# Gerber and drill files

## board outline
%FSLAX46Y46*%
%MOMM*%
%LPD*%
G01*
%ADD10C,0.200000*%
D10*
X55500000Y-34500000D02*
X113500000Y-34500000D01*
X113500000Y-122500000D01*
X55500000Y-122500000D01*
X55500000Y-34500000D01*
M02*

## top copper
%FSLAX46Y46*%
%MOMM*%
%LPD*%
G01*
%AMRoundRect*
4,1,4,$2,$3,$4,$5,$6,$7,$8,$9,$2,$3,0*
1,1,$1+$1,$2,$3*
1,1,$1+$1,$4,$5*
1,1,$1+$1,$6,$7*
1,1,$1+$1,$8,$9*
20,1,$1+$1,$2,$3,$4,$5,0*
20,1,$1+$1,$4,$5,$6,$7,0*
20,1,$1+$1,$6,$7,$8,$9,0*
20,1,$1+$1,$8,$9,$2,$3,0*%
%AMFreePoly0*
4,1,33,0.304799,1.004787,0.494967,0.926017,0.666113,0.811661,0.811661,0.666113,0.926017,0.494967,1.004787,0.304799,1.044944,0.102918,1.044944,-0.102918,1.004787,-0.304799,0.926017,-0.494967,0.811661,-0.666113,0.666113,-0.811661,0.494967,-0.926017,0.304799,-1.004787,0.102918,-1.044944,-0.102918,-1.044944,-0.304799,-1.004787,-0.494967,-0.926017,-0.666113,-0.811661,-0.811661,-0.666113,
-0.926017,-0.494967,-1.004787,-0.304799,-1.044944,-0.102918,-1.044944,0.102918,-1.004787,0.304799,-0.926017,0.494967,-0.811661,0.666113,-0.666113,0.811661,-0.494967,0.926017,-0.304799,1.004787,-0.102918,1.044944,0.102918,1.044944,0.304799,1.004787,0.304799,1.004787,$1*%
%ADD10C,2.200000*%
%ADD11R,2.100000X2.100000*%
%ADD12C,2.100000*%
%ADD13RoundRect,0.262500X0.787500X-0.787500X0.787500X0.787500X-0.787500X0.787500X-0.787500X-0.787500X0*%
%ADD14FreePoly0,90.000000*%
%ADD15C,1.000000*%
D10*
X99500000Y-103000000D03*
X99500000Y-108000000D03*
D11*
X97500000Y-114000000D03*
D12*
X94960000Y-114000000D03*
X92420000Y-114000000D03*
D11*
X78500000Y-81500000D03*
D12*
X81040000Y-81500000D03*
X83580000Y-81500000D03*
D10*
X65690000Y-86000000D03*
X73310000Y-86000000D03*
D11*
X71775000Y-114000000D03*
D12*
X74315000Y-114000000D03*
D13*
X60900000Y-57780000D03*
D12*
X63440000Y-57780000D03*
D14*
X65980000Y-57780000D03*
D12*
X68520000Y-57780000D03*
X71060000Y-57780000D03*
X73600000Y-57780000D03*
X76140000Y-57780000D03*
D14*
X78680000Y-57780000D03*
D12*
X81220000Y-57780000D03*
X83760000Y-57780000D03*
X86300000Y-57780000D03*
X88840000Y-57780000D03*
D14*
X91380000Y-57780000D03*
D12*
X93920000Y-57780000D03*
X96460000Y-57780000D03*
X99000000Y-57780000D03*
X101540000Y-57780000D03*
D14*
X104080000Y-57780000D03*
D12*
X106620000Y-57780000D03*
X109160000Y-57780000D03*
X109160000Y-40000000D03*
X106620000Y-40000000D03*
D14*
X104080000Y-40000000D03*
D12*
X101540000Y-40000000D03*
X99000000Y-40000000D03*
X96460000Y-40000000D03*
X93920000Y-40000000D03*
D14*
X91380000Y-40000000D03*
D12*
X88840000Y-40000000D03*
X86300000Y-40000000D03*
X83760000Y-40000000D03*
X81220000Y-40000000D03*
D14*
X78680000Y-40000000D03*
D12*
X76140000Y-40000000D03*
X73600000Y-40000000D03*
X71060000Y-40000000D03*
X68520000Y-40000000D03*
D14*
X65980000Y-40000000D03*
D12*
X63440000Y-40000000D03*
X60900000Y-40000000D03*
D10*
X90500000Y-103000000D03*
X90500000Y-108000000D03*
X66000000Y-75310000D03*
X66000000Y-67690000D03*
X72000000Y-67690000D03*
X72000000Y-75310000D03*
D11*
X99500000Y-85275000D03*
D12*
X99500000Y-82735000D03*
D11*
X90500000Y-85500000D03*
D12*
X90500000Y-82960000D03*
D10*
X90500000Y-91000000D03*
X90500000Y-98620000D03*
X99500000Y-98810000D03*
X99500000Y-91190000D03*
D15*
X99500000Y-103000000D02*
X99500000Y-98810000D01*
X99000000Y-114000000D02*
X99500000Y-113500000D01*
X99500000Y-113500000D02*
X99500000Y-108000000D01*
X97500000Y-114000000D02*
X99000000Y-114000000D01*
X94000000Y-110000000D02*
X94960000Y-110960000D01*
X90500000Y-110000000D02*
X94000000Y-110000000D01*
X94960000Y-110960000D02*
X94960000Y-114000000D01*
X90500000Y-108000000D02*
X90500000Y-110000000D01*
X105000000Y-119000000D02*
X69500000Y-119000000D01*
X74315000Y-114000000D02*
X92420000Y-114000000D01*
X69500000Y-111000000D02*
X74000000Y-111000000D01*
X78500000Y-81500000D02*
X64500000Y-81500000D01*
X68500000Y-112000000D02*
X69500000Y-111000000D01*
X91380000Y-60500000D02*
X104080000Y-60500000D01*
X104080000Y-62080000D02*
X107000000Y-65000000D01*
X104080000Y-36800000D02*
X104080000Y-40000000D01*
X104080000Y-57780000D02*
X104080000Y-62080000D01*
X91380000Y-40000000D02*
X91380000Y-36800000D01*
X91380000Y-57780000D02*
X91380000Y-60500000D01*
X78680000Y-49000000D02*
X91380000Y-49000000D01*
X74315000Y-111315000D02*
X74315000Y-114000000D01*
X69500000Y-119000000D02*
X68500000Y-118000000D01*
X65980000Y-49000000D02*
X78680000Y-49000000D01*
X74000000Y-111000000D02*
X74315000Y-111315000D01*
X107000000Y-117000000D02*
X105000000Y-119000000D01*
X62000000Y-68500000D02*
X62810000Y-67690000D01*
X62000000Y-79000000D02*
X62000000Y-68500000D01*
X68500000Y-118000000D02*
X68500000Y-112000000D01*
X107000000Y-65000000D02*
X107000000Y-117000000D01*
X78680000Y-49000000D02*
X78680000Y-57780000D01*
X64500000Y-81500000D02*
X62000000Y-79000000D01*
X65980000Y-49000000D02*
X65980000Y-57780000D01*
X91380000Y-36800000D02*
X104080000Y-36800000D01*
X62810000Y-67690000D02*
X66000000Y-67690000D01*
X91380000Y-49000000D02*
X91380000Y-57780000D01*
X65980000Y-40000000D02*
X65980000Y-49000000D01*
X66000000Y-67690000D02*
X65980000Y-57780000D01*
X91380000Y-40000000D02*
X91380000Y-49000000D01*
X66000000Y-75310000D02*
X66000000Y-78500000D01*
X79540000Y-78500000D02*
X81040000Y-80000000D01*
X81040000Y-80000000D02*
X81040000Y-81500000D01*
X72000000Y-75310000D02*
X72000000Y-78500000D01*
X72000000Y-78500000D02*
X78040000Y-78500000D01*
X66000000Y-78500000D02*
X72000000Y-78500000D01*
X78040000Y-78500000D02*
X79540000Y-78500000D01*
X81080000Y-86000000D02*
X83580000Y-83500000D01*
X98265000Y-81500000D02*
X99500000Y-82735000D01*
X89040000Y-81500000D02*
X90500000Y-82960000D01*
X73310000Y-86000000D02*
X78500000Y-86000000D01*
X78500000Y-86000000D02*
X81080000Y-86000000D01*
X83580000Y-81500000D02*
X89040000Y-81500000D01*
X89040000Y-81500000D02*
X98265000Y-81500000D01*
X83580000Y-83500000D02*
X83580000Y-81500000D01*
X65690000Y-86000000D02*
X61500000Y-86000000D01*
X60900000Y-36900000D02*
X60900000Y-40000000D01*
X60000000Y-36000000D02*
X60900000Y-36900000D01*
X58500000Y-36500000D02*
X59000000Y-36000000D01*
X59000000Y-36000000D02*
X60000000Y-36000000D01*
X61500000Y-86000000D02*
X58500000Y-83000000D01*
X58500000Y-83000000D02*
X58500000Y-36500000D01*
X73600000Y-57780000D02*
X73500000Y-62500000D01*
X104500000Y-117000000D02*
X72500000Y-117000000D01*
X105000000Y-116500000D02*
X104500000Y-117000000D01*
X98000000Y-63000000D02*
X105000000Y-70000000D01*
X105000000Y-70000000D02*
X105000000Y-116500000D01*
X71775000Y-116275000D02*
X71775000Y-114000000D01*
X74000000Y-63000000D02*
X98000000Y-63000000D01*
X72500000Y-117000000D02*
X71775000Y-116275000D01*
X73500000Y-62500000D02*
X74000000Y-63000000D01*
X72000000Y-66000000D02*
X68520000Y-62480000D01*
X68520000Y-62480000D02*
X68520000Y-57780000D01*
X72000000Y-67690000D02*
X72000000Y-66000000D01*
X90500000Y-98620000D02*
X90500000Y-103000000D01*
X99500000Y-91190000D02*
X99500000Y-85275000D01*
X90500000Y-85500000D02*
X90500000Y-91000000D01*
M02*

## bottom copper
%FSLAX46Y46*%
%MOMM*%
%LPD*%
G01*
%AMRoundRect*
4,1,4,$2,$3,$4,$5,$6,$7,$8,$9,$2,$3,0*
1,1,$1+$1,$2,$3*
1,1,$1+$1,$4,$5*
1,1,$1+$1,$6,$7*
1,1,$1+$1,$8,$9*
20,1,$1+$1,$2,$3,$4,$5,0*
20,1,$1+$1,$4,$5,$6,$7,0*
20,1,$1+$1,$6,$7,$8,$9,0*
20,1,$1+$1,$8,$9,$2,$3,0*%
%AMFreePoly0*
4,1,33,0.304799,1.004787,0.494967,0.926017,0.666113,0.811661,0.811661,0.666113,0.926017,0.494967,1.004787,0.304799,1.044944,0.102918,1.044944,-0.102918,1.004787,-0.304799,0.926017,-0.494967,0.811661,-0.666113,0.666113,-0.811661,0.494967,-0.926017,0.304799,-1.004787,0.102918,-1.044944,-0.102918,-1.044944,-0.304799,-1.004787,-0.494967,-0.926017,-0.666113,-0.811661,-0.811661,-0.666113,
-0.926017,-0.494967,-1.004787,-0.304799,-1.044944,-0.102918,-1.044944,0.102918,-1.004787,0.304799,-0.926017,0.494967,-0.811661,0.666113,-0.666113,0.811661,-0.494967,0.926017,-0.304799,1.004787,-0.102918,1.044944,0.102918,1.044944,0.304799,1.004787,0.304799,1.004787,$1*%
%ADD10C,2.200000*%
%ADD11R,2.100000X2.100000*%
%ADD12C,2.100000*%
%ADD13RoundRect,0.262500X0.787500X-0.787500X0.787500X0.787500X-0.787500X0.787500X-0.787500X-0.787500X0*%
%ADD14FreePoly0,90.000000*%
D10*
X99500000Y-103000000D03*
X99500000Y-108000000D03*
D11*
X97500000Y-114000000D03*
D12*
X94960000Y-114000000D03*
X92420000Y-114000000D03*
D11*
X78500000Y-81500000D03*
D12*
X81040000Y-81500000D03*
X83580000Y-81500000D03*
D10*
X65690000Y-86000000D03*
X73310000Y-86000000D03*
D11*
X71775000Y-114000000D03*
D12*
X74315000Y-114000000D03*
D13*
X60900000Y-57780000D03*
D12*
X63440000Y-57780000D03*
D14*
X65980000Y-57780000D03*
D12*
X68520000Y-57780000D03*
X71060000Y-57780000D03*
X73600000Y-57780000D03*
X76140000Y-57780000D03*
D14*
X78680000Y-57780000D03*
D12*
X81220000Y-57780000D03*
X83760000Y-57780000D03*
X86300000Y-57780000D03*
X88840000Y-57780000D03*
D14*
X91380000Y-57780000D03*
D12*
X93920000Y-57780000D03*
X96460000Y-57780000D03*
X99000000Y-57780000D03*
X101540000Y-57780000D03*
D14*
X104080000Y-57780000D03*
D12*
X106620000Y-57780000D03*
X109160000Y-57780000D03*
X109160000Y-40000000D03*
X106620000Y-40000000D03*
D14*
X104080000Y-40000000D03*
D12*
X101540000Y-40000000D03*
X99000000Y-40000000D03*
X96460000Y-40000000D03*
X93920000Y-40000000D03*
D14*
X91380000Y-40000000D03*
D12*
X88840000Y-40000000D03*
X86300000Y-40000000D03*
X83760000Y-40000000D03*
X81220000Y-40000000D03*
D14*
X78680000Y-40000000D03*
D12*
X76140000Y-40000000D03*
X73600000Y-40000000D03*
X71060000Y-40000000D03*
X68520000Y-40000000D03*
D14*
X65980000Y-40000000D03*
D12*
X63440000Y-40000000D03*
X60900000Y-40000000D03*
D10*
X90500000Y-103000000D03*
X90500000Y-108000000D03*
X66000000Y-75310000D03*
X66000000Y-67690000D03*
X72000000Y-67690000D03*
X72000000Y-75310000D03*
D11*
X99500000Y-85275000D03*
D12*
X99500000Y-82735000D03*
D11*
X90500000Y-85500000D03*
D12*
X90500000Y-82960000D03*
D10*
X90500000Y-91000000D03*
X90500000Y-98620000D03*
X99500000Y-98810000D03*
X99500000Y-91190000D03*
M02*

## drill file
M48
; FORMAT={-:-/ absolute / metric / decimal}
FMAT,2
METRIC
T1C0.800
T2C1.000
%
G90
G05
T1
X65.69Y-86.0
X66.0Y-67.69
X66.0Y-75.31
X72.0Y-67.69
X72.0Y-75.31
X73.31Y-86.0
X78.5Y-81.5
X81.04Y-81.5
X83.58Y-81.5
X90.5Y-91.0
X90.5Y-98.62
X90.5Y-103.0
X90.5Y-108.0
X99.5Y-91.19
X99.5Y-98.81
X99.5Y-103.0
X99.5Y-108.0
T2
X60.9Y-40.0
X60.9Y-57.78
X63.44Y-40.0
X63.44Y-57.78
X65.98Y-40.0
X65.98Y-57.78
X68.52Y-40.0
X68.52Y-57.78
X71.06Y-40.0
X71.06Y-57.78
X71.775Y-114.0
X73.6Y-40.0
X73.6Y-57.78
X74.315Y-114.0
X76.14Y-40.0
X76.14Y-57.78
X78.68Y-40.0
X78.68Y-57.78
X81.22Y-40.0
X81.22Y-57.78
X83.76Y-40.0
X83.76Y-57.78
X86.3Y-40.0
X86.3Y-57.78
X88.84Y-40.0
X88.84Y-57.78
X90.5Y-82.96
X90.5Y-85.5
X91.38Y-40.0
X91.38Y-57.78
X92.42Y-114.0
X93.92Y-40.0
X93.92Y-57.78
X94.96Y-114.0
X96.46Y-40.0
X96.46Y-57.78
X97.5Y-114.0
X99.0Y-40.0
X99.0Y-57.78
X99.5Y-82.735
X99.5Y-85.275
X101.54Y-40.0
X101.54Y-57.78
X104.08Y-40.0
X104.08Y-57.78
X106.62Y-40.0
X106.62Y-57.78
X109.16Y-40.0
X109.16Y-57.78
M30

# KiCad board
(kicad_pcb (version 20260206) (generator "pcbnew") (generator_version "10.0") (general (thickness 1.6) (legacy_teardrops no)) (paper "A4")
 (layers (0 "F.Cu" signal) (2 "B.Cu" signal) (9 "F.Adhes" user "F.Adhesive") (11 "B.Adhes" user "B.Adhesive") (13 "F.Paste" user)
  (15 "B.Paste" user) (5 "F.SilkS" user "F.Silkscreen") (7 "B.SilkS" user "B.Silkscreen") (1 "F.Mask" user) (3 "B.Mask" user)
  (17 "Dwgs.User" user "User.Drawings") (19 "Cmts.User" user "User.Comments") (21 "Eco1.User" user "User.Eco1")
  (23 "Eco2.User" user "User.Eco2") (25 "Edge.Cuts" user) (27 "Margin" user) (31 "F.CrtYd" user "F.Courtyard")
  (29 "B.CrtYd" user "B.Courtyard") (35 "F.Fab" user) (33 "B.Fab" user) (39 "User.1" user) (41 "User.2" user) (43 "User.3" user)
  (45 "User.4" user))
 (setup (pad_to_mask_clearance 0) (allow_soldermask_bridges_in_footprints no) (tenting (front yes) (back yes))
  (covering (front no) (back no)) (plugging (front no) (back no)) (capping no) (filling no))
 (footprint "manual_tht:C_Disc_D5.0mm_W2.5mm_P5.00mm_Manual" (layer "F.Cu") (at 99.5 103 -90)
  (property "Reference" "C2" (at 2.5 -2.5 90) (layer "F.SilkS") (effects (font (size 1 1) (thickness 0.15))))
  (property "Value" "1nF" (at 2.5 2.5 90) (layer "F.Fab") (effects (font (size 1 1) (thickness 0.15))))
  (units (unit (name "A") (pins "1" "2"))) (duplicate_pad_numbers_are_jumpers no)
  (pad "1" thru_hole circle (at 0 0 270) (size 2.2 2.2) (drill 0.8) (layers "*.Cu" "*.Mask") (remove_unused_layers no) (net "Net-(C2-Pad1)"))
  (pad "2" thru_hole circle (at 5 0 270) (size 2.2 2.2) (drill 0.8) (layers "*.Cu" "*.Mask") (remove_unused_layers no) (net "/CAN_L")))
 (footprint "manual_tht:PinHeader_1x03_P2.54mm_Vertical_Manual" (layer "F.Cu") (at 97.5 114 -90)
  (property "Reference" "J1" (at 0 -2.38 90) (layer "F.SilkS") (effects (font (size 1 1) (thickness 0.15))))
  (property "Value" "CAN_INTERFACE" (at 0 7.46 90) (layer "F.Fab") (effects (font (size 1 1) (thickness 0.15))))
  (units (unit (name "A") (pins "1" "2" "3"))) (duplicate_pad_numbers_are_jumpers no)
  (pad "1" thru_hole rect (at 0 0 270) (size 2.1 2.1) (drill 1) (layers "*.Cu" "*.Mask") (remove_unused_layers no) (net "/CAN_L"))
  (pad "2" thru_hole circle (at 0 2.54 270) (size 2.1 2.1) (drill 1) (layers "*.Cu" "*.Mask") (remove_unused_layers no) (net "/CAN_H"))
  (pad "3" thru_hole circle (at 0 5.08 270) (size 2.1 2.1) (drill 1) (layers "*.Cu" "*.Mask") (remove_unused_layers no) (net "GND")))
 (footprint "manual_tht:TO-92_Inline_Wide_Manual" (layer "F.Cu") (at 78.5 81.5)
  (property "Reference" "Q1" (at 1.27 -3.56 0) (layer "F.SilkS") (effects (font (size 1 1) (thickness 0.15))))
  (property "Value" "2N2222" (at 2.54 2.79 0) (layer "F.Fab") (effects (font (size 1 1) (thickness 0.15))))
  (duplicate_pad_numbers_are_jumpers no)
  (pad "1" thru_hole rect (at 0 0) (size 2.1 2.1) (drill 0.8) (layers "*.Cu" "*.Mask") (remove_unused_layers no) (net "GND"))
  (pad "2" thru_hole circle (at 2.54 0) (size 2.1 2.1) (drill 0.8) (layers "*.Cu" "*.Mask") (remove_unused_layers no) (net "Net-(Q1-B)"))
  (pad "3" thru_hole circle (at 5.08 0) (size 2.1 2.1) (drill 0.8) (layers "*.Cu" "*.Mask") (remove_unused_layers no) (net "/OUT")))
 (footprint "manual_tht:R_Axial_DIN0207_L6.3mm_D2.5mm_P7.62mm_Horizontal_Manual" (layer "F.Cu") (at 65.69 86)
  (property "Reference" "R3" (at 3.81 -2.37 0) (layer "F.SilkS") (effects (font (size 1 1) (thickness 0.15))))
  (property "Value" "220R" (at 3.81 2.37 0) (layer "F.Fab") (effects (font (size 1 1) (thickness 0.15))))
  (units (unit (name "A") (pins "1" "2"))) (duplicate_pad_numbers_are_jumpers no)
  (pad "1" thru_hole circle (at 0 0) (size 2.2 2.2) (drill 0.8) (layers "*.Cu" "*.Mask") (remove_unused_layers no) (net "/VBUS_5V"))
  (pad "2" thru_hole circle (at 7.62 0) (size 2.2 2.2) (drill 0.8) (layers "*.Cu" "*.Mask") (remove_unused_layers no) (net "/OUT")))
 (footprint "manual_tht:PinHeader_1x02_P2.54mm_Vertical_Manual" (layer "F.Cu") (at 71.775 114 90)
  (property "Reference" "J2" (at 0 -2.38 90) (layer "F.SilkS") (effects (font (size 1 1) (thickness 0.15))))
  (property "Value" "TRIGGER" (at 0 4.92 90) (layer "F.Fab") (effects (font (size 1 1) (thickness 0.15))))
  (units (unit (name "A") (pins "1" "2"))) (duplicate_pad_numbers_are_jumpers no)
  (pad "1" thru_hole rect (at 0 0 90) (size 2.1 2.1) (drill 1) (layers "*.Cu" "*.Mask") (remove_unused_layers no) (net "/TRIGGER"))
  (pad "2" thru_hole circle (at 0 2.54 90) (size 2.1 2.1) (drill 1) (layers "*.Cu" "*.Mask") (remove_unused_layers no) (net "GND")))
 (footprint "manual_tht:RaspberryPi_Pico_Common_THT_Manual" (layer "F.Cu") (at 60.9 57.78 90)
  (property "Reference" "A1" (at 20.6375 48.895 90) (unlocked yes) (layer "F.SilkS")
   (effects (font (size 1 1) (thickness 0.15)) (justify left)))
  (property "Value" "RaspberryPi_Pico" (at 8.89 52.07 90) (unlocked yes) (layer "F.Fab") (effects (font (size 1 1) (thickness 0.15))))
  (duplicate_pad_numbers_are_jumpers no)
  (pad "1" thru_hole roundrect (at 0 0 90) (size 2.1 2.1) (drill 1) (layers "*.Cu" "*.Mask") (remove_unused_layers no)
   (roundrect_rratio 0.125) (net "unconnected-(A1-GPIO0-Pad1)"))
  (pad "2" thru_hole circle (at 0 2.54 90) (size 2.1 2.1) (drill 1) (layers "*.Cu" "*.Mask") (remove_unused_layers no)
   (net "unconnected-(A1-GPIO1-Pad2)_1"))
  (pad "3" thru_hole custom (at 0 5.08 90) (size 2.1 2.1) (drill 1) (layers "*.Cu" "*.Mask") (remove_unused_layers no) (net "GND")
   (options (clearance outline) (anchor circle)) (primitives))
  (pad "4" thru_hole circle (at 0 7.62 90) (size 2.1 2.1) (drill 1) (layers "*.Cu" "*.Mask") (remove_unused_layers no) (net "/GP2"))
  (pad "5" thru_hole circle (at 0 10.16 90) (size 2.1 2.1) (drill 1) (layers "*.Cu" "*.Mask") (remove_unused_layers no)
   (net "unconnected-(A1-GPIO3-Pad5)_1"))
  (pad "6" thru_hole circle (at 0 12.7 90) (size 2.1 2.1) (drill 1) (layers "*.Cu" "*.Mask") (remove_unused_layers no) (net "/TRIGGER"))
  (pad "7" thru_hole circle (at 0 15.24 90) (size 2.1 2.1) (drill 1) (layers "*.Cu" "*.Mask") (remove_unused_layers no)
   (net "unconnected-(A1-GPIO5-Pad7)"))
  (pad "8" thru_hole custom (at 0 17.78 90) (size 2.1 2.1) (drill 1) (layers "*.Cu" "*.Mask") (remove_unused_layers no) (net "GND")
   (options (clearance outline) (anchor circle)) (primitives))
  (pad "9" thru_hole circle (at 0 20.32 90) (size 2.1 2.1) (drill 1) (layers "*.Cu" "*.Mask") (remove_unused_layers no)
   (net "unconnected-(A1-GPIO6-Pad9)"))
  (pad "10" thru_hole circle (at 0 22.86 90) (size 2.1 2.1) (drill 1) (layers "*.Cu" "*.Mask") (remove_unused_layers no)
   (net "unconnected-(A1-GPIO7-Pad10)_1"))
  (pad "11" thru_hole circle (at 0 25.4 90) (size 2.1 2.1) (drill 1) (layers "*.Cu" "*.Mask") (remove_unused_layers no)
   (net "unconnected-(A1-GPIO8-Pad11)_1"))
  (pad "12" thru_hole circle (at 0 27.94 90) (size 2.1 2.1) (drill 1) (layers "*.Cu" "*.Mask") (remove_unused_layers no)
   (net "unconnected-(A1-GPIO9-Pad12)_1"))
  (pad "13" thru_hole custom (at 0 30.48 90) (size 2.1 2.1) (drill 1) (layers "*.Cu" "*.Mask") (remove_unused_layers no) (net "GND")
   (options (clearance outline) (anchor circle)) (primitives))
  (pad "14" thru_hole circle (at 0 33.02 90) (size 2.1 2.1) (drill 1) (layers "*.Cu" "*.Mask") (remove_unused_layers no)
   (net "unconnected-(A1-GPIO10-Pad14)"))
  (pad "15" thru_hole circle (at 0 35.56 90) (size 2.1 2.1) (drill 1) (layers "*.Cu" "*.Mask") (remove_unused_layers no)
   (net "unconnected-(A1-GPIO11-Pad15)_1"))
  (pad "16" thru_hole circle (at 0 38.1 90) (size 2.1 2.1) (drill 1) (layers "*.Cu" "*.Mask") (remove_unused_layers no)
   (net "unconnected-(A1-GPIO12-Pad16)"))
  (pad "17" thru_hole circle (at 0 40.64 90) (size 2.1 2.1) (drill 1) (layers "*.Cu" "*.Mask") (remove_unused_layers no)
   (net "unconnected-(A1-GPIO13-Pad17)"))
  (pad "18" thru_hole custom (at 0 43.18 90) (size 2.1 2.1) (drill 1) (layers "*.Cu" "*.Mask") (remove_unused_layers no) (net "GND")
   (options (clearance outline) (anchor circle)) (primitives))
  (pad "19" thru_hole circle (at 0 45.72 90) (size 2.1 2.1) (drill 1) (layers "*.Cu" "*.Mask") (remove_unused_layers no)
   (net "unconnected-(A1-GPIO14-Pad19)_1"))
  (pad "20" thru_hole circle (at 0 48.26 90) (size 2.1 2.1) (drill 1) (layers "*.Cu" "*.Mask") (remove_unused_layers no)
   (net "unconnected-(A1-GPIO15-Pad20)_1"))
  (pad "21" thru_hole circle (at 17.78 48.26 90) (size 2.1 2.1) (drill 1) (layers "*.Cu" "*.Mask") (remove_unused_layers no)
   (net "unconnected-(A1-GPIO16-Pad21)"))
  (pad "22" thru_hole circle (at 17.78 45.72 90) (size 2.1 2.1) (drill 1) (layers "*.Cu" "*.Mask") (remove_unused_layers no)
   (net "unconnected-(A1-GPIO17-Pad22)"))
  (pad "23" thru_hole custom (at 17.78 43.18 90) (size 2.1 2.1) (drill 1) (layers "*.Cu" "*.Mask") (remove_unused_layers no) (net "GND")
   (options (clearance outline) (anchor circle)) (primitives))
  (pad "24" thru_hole circle (at 17.78 40.64 90) (size 2.1 2.1) (drill 1) (layers "*.Cu" "*.Mask") (remove_unused_layers no)
   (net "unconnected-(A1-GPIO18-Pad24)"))
  (pad "25" thru_hole circle (at 17.78 38.1 90) (size 2.1 2.1) (drill 1) (layers "*.Cu" "*.Mask") (remove_unused_layers no)
   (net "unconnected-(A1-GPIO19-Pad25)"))
  (pad "26" thru_hole circle (at 17.78 35.56 90) (size 2.1 2.1) (drill 1) (layers "*.Cu" "*.Mask") (remove_unused_layers no)
   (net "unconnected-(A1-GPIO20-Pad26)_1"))
  (pad "27" thru_hole circle (at 17.78 33.02 90) (size 2.1 2.1) (drill 1) (layers "*.Cu" "*.Mask") (remove_unused_layers no)
   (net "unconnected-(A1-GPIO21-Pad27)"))
  (pad "28" thru_hole custom (at 17.78 30.48 90) (size 2.1 2.1) (drill 1) (layers "*.Cu" "*.Mask") (remove_unused_layers no) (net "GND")
   (options (clearance outline) (anchor circle)) (primitives))
  (pad "29" thru_hole circle (at 17.78 27.94 90) (size 2.1 2.1) (drill 1) (layers "*.Cu" "*.Mask") (remove_unused_layers no)
   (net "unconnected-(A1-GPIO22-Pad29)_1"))
  (pad "30" thru_hole circle (at 17.78 25.4 90) (size 2.1 2.1) (drill 1) (layers "*.Cu" "*.Mask") (remove_unused_layers no)
   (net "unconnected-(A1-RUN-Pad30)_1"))
  (pad "31" thru_hole circle (at 17.78 22.86 90) (size 2.1 2.1) (drill 1) (layers "*.Cu" "*.Mask") (remove_unused_layers no)
   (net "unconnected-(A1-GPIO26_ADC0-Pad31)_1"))
  (pad "32" thru_hole circle (at 17.78 20.32 90) (size 2.1 2.1) (drill 1) (layers "*.Cu" "*.Mask") (remove_unused_layers no)
   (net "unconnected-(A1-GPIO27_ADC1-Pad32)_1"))
  (pad "33" thru_hole custom (at 17.78 17.78 90) (size 2.1 2.1) (drill 1) (layers "*.Cu" "*.Mask") (remove_unused_layers no)
   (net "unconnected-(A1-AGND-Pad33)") (options (clearance outline) (anchor circle)) (primitives))
  (pad "34" thru_hole circle (at 17.78 15.24 90) (size 2.1 2.1) (drill 1) (layers "*.Cu" "*.Mask") (remove_unused_layers no)
   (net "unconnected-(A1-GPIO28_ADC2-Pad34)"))
  (pad "35" thru_hole circle (at 17.78 12.7 90) (size 2.1 2.1) (drill 1) (layers "*.Cu" "*.Mask") (remove_unused_layers no)
   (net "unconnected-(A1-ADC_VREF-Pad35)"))
  (pad "36" thru_hole circle (at 17.78 10.16 90) (size 2.1 2.1) (drill 1) (layers "*.Cu" "*.Mask") (remove_unused_layers no)
   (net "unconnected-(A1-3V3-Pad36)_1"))
  (pad "37" thru_hole circle (at 17.78 7.62 90) (size 2.1 2.1) (drill 1) (layers "*.Cu" "*.Mask") (remove_unused_layers no)
   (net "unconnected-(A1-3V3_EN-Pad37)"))
  (pad "38" thru_hole custom (at 17.78 5.08 90) (size 2.1 2.1) (drill 1) (layers "*.Cu" "*.Mask") (remove_unused_layers no) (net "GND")
   (options (clearance outline) (anchor circle)) (primitives))
  (pad "39" thru_hole circle (at 17.78 2.54 90) (size 2.1 2.1) (drill 1) (layers "*.Cu" "*.Mask") (remove_unused_layers no)
   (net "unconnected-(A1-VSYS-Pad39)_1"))
  (pad "40" thru_hole circle (at 17.78 0 90) (size 2.1 2.1) (drill 1) (layers "*.Cu" "*.Mask") (remove_unused_layers no) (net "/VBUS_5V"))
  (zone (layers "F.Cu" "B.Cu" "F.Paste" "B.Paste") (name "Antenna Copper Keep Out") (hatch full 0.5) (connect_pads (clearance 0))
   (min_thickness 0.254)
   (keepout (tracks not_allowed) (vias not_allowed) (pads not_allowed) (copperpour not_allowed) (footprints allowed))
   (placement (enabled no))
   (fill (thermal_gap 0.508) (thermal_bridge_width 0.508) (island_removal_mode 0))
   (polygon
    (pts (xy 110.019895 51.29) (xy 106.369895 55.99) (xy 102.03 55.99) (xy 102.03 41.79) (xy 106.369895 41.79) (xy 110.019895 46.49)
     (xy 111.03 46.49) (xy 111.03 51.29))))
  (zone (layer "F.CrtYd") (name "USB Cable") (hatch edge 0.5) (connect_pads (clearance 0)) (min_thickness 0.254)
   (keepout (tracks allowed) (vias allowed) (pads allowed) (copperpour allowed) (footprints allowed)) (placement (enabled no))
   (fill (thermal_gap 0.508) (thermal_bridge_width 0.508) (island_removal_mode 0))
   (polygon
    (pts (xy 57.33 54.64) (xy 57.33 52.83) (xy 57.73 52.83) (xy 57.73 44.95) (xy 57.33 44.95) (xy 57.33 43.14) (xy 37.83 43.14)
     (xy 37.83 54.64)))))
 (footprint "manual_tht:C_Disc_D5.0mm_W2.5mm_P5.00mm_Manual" (layer "F.Cu") (at 90.5 103 -90)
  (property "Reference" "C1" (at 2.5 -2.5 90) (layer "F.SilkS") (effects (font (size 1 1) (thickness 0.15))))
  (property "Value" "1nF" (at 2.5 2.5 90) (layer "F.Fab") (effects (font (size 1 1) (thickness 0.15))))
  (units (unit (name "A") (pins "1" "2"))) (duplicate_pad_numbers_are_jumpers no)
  (pad "1" thru_hole circle (at 0 0 270) (size 2.2 2.2) (drill 0.8) (layers "*.Cu" "*.Mask") (remove_unused_layers no) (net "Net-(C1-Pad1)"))
  (pad "2" thru_hole circle (at 5 0 270) (size 2.2 2.2) (drill 0.8) (layers "*.Cu" "*.Mask") (remove_unused_layers no) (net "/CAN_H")))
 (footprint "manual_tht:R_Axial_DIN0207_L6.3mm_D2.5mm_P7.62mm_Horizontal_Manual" (layer "F.Cu") (at 66 75.31 90)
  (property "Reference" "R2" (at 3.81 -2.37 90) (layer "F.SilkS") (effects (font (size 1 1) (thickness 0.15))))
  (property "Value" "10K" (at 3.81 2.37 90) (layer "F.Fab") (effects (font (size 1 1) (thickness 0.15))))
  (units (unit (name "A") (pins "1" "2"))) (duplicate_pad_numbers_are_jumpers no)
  (pad "1" thru_hole circle (at 0 0 90) (size 2.2 2.2) (drill 0.8) (layers "*.Cu" "*.Mask") (remove_unused_layers no) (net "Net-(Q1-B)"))
  (pad "2" thru_hole circle (at 7.62 0 90) (size 2.2 2.2) (drill 0.8) (layers "*.Cu" "*.Mask") (remove_unused_layers no) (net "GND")))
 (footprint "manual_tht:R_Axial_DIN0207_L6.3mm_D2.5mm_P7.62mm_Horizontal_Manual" (layer "F.Cu") (at 72 67.69 -90)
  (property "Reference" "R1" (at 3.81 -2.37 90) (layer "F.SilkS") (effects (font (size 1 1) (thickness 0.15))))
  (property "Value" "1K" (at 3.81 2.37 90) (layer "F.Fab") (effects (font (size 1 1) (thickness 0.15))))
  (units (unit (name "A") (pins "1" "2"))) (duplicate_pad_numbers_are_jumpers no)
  (pad "1" thru_hole circle (at 0 0 270) (size 2.2 2.2) (drill 0.8) (layers "*.Cu" "*.Mask") (remove_unused_layers no) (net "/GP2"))
  (pad "2" thru_hole circle (at 7.62 0 270) (size 2.2 2.2) (drill 0.8) (layers "*.Cu" "*.Mask") (remove_unused_layers no) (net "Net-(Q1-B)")))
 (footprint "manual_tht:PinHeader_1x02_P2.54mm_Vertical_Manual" (layer "F.Cu") (at 99.5 85.275 180)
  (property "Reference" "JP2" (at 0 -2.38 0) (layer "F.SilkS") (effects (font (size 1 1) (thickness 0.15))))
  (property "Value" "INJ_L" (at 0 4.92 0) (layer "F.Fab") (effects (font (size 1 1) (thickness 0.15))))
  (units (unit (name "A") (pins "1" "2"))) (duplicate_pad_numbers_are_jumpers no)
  (pad "1" thru_hole rect (at 0 0 180) (size 2.1 2.1) (drill 1) (layers "*.Cu" "*.Mask") (remove_unused_layers no) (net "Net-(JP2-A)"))
  (pad "2" thru_hole circle (at 0 2.54 180) (size 2.1 2.1) (drill 1) (layers "*.Cu" "*.Mask") (remove_unused_layers no) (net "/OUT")))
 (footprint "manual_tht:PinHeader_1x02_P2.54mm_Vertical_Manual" (layer "F.Cu") (at 90.5 85.5 180)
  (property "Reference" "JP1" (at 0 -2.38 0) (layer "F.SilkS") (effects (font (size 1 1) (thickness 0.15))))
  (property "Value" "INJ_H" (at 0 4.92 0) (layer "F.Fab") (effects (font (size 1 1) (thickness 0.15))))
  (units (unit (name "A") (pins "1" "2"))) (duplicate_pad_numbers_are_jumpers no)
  (pad "1" thru_hole rect (at 0 0 180) (size 2.1 2.1) (drill 1) (layers "*.Cu" "*.Mask") (remove_unused_layers no) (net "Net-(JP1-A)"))
  (pad "2" thru_hole circle (at 0 2.54 180) (size 2.1 2.1) (drill 1) (layers "*.Cu" "*.Mask") (remove_unused_layers no) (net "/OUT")))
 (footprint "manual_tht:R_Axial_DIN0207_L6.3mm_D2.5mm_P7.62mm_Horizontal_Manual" (layer "F.Cu") (at 90.5 91 -90)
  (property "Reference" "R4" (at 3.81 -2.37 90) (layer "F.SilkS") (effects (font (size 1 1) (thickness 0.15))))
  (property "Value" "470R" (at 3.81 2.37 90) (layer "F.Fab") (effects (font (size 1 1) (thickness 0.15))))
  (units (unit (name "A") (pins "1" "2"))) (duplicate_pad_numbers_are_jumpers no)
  (pad "1" thru_hole circle (at 0 0 270) (size 2.2 2.2) (drill 0.8) (layers "*.Cu" "*.Mask") (remove_unused_layers no) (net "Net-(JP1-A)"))
  (pad "2" thru_hole circle (at 7.62 0 270) (size 2.2 2.2) (drill 0.8) (layers "*.Cu" "*.Mask") (remove_unused_layers no)
   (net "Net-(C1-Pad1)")))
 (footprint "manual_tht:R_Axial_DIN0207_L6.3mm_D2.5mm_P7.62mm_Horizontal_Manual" (layer "F.Cu") (at 99.5 98.81 90)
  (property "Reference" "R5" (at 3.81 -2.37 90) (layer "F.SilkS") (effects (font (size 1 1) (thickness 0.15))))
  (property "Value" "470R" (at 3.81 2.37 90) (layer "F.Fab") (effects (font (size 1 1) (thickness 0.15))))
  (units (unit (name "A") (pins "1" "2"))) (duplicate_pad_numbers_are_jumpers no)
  (pad "1" thru_hole circle (at 0 0 90) (size 2.2 2.2) (drill 0.8) (layers "*.Cu" "*.Mask") (remove_unused_layers no) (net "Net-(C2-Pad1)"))
  (pad "2" thru_hole circle (at 7.62 0 90) (size 2.2 2.2) (drill 0.8) (layers "*.Cu" "*.Mask") (remove_unused_layers no) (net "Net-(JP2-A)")))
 (gr_rect (start 55.5 34.5) (end 113.5 122.5) (stroke (width 0.2) (type default)) (fill no) (layer "Edge.Cuts"))
 (segment (start 99.5 103) (end 99.5 98.81) (width 1) (layer "F.Cu") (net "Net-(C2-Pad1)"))
 (segment (start 99 114) (end 99.5 113.5) (width 1) (layer "F.Cu") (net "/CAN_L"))
 (segment (start 99.5 113.5) (end 99.5 108) (width 1) (layer "F.Cu") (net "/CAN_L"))
 (segment (start 97.5 114) (end 99 114) (width 1) (layer "F.Cu") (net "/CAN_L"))
 (segment (start 94 110) (end 94.96 110.96) (width 1) (layer "F.Cu") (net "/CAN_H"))
 (segment (start 90.5 110) (end 94 110) (width 1) (layer "F.Cu") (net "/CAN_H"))
 (segment (start 94.96 110.96) (end 94.96 114) (width 1) (layer "F.Cu") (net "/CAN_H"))
 (segment (start 90.5 108) (end 90.5 110) (width 1) (layer "F.Cu") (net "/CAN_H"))
 (segment (start 105 119) (end 69.5 119) (width 1) (layer "F.Cu") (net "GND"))
 (segment (start 74.315 114) (end 92.42 114) (width 1) (layer "F.Cu") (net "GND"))
 (segment (start 69.5 111) (end 74 111) (width 1) (layer "F.Cu") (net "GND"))
 (segment (start 78.5 81.5) (end 64.5 81.5) (width 1) (layer "F.Cu") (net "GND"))
 (segment (start 68.5 112) (end 69.5 111) (width 1) (layer "F.Cu") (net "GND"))
 (segment (start 91.38 60.5) (end 104.08 60.5) (width 1) (layer "F.Cu") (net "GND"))
 (segment (start 104.08 62.08) (end 107 65) (width 1) (layer "F.Cu") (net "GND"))
 (segment (start 104.08 36.8) (end 104.08 40) (width 1) (layer "F.Cu") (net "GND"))
 (segment (start 104.08 57.78) (end 104.08 62.08) (width 1) (layer "F.Cu") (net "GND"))
 (segment (start 91.38 40) (end 91.38 36.8) (width 1) (layer "F.Cu") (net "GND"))
 (segment (start 91.38 57.78) (end 91.38 60.5) (width 1) (layer "F.Cu") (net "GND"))
 (segment (start 78.68 49) (end 91.38 49) (width 1) (layer "F.Cu") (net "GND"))
 (segment (start 74.315 111.315) (end 74.315 114) (width 1) (layer "F.Cu") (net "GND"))
 (segment (start 69.5 119) (end 68.5 118) (width 1) (layer "F.Cu") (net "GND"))
 (segment (start 65.98 49) (end 78.68 49) (width 1) (layer "F.Cu") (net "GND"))
 (segment (start 74 111) (end 74.315 111.315) (width 1) (layer "F.Cu") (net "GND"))
 (segment (start 107 117) (end 105 119) (width 1) (layer "F.Cu") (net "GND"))
 (segment (start 62 68.5) (end 62.81 67.69) (width 1) (layer "F.Cu") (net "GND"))
 (segment (start 62 79) (end 62 68.5) (width 1) (layer "F.Cu") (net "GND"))
 (segment (start 68.5 118) (end 68.5 112) (width 1) (layer "F.Cu") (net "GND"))
 (segment (start 107 65) (end 107 117) (width 1) (layer "F.Cu") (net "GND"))
 (segment (start 78.68 49) (end 78.68 57.78) (width 1) (layer "F.Cu") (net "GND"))
 (segment (start 64.5 81.5) (end 62 79) (width 1) (layer "F.Cu") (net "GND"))
 (segment (start 65.98 49) (end 65.98 57.78) (width 1) (layer "F.Cu") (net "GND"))
 (segment (start 91.38 36.8) (end 104.08 36.8) (width 1) (layer "F.Cu") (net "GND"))
 (segment (start 62.81 67.69) (end 66 67.69) (width 1) (layer "F.Cu") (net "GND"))
 (segment (start 91.38 49) (end 91.38 57.78) (width 1) (layer "F.Cu") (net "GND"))
 (segment (start 65.98 40) (end 65.98 49) (width 1) (layer "F.Cu") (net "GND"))
 (segment (start 66 67.69) (end 65.98 57.78) (width 1) (layer "F.Cu") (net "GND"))
 (segment (start 91.38 40) (end 91.38 49) (width 1) (layer "F.Cu") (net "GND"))
 (segment (start 66 75.31) (end 66 78.5) (width 1) (layer "F.Cu") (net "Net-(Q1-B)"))
 (segment (start 79.54 78.5) (end 81.04 80) (width 1) (layer "F.Cu") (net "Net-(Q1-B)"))
 (segment (start 81.04 80) (end 81.04 81.5) (width 1) (layer "F.Cu") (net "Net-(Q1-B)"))
 (segment (start 72 75.31) (end 72 78.5) (width 1) (layer "F.Cu") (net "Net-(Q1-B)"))
 (segment (start 72 78.5) (end 78.04 78.5) (width 1) (layer "F.Cu") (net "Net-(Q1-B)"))
 (segment (start 66 78.5) (end 72 78.5) (width 1) (layer "F.Cu") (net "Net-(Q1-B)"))
 (segment (start 78.04 78.5) (end 79.54 78.5) (width 1) (layer "F.Cu") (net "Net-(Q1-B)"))
 (segment (start 81.08 86) (end 83.58 83.5) (width 1) (layer "F.Cu") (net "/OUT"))
 (segment (start 98.265 81.5) (end 99.5 82.735) (width 1) (layer "F.Cu") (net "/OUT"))
 (segment (start 89.04 81.5) (end 90.5 82.96) (width 1) (layer "F.Cu") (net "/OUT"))
 (segment (start 73.31 86) (end 78.5 86) (width 1) (layer "F.Cu") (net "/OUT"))
 (segment (start 78.5 86) (end 81.08 86) (width 1) (layer "F.Cu") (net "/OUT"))
 (segment (start 83.58 81.5) (end 89.04 81.5) (width 1) (layer "F.Cu") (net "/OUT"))
 (segment (start 89.04 81.5) (end 98.265 81.5) (width 1) (layer "F.Cu") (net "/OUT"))
 (segment (start 83.58 83.5) (end 83.58 81.5) (width 1) (layer "F.Cu") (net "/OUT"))
 (segment (start 65.69 86) (end 61.5 86) (width 1) (layer "F.Cu") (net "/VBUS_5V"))
 (segment (start 60.9 36.9) (end 60.9 40) (width 1) (layer "F.Cu") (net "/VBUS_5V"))
 (segment (start 60 36) (end 60.9 36.9) (width 1) (layer "F.Cu") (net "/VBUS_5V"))
 (segment (start 58.5 36.5) (end 59 36) (width 1) (layer "F.Cu") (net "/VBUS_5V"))
 (segment (start 59 36) (end 60 36) (width 1) (layer "F.Cu") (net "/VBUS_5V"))
 (segment (start 61.5 86) (end 58.5 83) (width 1) (layer "F.Cu") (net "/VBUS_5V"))
 (segment (start 58.5 83) (end 58.5 36.5) (width 1) (layer "F.Cu") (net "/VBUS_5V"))
 (segment (start 73.6 57.78) (end 73.5 62.5) (width 1) (layer "F.Cu") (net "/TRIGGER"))
 (segment (start 104.5 117) (end 72.5 117) (width 1) (layer "F.Cu") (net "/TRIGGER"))
 (segment (start 105 116.5) (end 104.5 117) (width 1) (layer "F.Cu") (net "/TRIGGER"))
 (segment (start 98 63) (end 105 70) (width 1) (layer "F.Cu") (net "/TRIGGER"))
 (segment (start 105 70) (end 105 116.5) (width 1) (layer "F.Cu") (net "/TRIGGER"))
 (segment (start 71.775 116.275) (end 71.775 114) (width 1) (layer "F.Cu") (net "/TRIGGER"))
 (segment (start 74 63) (end 98 63) (width 1) (layer "F.Cu") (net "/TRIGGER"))
 (segment (start 72.5 117) (end 71.775 116.275) (width 1) (layer "F.Cu") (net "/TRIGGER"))
 (segment (start 73.5 62.5) (end 74 63) (width 1) (layer "F.Cu") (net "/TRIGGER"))
 (segment (start 72 66) (end 68.52 62.48) (width 1) (layer "F.Cu") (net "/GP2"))
 (segment (start 68.52 62.48) (end 68.52 57.78) (width 1) (layer "F.Cu") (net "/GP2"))
 (segment (start 72 67.69) (end 72 66) (width 1) (layer "F.Cu") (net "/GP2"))
 (segment (start 90.5 98.62) (end 90.5 103) (width 1) (layer "F.Cu") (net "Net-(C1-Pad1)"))
 (segment (start 99.5 91.19) (end 99.5 85.275) (width 1) (layer "F.Cu") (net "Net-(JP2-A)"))
 (segment (start 90.5 85.5) (end 90.5 91) (width 1) (layer "F.Cu") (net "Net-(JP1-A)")))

